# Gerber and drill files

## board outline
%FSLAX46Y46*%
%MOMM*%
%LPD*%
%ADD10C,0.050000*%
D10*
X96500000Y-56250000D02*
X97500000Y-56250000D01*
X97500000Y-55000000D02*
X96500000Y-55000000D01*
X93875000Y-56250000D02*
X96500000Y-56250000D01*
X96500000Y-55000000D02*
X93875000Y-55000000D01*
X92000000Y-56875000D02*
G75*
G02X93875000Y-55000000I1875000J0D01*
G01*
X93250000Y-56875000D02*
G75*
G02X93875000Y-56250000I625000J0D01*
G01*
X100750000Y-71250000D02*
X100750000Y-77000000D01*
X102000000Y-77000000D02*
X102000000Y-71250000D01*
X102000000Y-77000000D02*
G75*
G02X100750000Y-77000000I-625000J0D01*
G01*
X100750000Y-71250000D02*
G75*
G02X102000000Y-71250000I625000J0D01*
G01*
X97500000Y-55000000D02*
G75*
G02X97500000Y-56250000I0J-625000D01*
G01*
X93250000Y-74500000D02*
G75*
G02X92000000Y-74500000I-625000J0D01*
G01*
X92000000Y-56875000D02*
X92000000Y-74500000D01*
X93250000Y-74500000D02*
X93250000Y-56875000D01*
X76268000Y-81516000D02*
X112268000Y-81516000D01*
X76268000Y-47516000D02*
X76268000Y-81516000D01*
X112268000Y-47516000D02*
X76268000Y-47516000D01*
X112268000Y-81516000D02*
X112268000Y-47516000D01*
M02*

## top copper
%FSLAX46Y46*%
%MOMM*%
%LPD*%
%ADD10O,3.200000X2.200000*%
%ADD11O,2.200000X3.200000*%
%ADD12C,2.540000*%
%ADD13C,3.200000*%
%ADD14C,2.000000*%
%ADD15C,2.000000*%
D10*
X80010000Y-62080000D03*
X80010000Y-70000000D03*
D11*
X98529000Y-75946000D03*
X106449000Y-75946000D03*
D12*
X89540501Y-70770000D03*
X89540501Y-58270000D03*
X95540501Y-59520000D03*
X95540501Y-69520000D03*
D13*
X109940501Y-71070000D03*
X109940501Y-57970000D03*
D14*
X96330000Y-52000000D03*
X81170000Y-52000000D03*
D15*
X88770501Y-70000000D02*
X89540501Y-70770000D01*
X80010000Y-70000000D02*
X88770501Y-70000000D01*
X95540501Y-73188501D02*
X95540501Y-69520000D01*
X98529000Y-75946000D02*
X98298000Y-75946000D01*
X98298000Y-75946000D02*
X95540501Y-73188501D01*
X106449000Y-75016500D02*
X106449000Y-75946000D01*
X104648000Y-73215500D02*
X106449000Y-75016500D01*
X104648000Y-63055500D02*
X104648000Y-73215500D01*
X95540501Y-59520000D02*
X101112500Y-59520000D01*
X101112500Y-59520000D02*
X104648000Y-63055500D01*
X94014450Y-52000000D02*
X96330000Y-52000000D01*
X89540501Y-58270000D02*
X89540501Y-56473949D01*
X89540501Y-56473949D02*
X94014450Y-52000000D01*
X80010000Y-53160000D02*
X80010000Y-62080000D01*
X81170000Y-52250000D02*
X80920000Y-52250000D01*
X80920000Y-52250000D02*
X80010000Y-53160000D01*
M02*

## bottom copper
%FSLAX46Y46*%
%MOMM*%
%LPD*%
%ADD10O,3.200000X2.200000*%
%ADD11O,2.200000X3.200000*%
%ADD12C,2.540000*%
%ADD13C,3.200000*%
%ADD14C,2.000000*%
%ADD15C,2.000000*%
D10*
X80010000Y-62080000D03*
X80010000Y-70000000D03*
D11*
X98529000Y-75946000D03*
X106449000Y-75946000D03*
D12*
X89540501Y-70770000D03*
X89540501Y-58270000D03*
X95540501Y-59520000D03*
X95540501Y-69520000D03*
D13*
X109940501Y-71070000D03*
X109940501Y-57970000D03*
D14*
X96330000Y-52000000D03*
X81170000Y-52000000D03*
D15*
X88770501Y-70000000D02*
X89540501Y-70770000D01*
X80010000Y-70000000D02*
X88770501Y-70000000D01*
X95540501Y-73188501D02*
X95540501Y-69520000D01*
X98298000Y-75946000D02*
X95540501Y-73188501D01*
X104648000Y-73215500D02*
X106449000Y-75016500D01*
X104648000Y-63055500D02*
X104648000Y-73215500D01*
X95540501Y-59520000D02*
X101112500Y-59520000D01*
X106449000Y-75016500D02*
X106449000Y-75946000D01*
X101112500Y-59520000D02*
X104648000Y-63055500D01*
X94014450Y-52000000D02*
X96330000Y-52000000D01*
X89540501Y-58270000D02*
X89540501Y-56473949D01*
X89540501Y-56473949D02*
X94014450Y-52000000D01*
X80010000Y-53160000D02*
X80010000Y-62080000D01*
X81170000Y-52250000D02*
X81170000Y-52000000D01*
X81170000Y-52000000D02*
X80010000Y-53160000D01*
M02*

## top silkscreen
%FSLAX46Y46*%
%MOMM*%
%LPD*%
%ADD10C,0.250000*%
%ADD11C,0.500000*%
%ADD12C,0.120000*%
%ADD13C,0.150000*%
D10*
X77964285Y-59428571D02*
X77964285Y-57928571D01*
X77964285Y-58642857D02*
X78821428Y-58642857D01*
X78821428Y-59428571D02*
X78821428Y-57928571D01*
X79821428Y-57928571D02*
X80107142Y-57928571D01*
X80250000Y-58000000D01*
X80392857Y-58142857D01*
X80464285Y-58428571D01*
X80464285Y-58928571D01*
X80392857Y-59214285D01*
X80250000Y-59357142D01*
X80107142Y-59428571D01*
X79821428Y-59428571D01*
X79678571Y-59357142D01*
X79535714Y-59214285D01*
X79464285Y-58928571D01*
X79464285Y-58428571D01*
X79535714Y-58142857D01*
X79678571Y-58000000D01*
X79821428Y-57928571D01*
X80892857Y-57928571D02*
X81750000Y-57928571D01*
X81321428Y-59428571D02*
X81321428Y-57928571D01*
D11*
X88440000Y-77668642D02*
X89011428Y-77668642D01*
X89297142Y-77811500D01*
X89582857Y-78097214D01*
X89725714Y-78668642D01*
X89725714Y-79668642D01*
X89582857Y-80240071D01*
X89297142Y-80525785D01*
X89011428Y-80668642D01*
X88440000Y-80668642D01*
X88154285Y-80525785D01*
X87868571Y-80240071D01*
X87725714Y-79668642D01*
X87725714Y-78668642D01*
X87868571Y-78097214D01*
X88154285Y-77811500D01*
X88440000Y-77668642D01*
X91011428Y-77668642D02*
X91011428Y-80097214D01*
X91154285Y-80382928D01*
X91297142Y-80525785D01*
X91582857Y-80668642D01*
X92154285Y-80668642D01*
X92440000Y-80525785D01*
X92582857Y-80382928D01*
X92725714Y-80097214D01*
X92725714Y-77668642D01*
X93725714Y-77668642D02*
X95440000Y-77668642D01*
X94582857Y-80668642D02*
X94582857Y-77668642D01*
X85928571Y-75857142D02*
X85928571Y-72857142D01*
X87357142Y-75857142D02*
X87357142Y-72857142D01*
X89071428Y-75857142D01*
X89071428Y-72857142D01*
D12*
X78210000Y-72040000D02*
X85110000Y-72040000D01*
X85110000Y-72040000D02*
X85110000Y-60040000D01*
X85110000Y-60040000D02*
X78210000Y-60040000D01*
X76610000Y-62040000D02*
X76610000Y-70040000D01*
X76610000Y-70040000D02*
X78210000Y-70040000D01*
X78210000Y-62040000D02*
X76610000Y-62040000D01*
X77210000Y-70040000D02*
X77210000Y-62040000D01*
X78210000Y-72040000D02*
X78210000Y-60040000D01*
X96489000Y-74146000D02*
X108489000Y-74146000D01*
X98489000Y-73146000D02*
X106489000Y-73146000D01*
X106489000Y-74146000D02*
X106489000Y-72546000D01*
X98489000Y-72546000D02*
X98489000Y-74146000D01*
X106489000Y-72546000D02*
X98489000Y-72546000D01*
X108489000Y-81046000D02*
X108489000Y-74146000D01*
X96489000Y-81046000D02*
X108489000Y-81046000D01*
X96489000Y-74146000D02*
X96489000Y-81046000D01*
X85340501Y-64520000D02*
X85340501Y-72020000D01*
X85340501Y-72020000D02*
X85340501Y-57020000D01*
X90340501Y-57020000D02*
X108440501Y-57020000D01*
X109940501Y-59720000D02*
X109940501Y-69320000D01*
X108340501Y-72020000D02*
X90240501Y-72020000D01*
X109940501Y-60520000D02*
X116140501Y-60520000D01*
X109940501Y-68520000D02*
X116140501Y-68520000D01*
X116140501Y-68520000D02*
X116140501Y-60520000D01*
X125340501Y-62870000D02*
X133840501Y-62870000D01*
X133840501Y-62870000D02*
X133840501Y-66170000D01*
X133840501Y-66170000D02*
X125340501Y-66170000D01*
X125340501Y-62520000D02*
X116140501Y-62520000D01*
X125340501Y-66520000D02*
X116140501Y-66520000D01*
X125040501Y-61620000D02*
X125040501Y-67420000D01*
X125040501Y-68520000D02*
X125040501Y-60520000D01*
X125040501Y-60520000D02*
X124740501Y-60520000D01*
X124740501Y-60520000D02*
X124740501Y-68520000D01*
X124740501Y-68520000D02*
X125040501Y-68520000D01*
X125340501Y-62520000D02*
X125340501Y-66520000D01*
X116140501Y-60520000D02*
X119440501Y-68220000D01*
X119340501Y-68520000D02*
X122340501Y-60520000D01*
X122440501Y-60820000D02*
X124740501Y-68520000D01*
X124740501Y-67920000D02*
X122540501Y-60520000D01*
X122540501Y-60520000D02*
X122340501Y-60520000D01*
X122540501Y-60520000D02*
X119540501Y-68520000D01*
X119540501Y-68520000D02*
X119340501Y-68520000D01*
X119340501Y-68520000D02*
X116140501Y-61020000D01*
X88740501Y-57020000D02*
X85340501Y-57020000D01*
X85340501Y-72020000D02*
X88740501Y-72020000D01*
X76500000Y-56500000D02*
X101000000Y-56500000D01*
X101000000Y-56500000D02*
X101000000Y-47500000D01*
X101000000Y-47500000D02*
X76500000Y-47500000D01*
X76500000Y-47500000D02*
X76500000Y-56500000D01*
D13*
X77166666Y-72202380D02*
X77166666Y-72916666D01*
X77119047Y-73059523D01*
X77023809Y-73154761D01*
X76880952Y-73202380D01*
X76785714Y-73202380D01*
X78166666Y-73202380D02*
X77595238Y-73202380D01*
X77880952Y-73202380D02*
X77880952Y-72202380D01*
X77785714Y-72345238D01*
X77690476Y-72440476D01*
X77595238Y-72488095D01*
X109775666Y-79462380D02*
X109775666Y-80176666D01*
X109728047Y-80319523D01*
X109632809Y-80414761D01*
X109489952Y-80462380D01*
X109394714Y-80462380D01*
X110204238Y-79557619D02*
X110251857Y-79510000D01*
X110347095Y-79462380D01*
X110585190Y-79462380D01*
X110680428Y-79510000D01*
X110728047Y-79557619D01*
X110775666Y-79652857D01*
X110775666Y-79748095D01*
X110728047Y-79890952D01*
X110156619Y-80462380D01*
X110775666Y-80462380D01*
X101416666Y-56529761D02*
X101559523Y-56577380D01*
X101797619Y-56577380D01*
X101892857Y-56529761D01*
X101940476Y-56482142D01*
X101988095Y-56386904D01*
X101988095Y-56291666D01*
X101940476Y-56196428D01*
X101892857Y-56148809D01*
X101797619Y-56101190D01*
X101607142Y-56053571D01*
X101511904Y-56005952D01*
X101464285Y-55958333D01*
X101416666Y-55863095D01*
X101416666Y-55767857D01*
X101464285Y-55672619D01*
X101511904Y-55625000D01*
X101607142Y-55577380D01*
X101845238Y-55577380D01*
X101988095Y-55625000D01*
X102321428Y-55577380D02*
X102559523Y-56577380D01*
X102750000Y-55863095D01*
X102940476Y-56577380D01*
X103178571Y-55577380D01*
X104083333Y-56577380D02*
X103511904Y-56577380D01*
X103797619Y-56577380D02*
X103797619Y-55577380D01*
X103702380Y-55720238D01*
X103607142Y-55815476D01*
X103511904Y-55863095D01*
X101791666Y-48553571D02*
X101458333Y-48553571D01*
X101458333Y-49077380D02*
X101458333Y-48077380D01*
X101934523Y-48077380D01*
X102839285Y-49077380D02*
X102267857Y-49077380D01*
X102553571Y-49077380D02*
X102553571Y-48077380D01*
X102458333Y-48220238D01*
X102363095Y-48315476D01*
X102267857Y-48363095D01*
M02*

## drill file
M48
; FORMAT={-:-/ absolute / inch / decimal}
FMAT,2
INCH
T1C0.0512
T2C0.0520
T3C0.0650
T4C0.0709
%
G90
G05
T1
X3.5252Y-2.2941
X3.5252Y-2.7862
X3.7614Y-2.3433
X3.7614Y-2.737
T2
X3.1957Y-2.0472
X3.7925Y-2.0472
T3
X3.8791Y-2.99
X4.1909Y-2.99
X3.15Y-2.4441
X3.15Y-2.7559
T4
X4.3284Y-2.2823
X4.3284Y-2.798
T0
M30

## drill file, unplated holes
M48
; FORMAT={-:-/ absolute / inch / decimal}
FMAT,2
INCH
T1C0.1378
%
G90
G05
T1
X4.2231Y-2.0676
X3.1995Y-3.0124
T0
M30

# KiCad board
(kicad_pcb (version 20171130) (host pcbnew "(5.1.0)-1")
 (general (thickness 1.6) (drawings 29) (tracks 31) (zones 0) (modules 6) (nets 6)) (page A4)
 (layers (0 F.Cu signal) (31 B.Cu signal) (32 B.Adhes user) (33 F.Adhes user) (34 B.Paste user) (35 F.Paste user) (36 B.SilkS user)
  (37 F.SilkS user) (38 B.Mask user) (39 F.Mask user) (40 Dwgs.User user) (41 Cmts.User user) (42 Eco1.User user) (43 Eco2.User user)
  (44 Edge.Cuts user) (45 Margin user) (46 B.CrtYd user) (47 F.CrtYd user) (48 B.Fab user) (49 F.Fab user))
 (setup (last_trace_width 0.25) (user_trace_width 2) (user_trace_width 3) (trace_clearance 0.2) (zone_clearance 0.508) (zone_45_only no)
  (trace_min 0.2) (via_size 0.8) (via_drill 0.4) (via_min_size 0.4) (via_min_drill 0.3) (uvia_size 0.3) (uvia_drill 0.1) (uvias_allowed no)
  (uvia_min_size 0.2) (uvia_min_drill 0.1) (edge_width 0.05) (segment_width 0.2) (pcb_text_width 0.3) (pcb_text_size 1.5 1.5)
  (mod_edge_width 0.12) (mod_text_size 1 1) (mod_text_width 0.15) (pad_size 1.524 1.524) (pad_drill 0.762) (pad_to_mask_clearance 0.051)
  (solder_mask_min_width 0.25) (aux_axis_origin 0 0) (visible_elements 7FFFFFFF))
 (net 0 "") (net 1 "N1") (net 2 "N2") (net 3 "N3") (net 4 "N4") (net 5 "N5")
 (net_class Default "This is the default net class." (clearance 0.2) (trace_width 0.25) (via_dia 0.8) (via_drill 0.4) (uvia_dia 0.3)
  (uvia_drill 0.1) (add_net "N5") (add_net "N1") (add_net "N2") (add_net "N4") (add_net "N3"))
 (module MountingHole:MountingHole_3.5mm (layer F.Cu) (at 107.268 52.516)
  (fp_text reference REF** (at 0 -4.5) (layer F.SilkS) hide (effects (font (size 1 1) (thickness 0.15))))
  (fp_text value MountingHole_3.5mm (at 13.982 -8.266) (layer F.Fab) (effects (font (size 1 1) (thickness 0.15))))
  (pad 1 np_thru_hole circle (at 0 0) (size 3.5 3.5) (drill 3.5) (layers *.Cu *.Mask)))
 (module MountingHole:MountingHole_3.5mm (layer F.Cu) (at 81.268 76.516)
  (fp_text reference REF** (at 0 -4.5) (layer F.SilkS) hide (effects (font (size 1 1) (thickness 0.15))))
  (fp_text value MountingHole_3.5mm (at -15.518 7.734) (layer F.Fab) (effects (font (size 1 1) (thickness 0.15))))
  (pad 1 np_thru_hole circle (at 0 0) (size 3.5 3.5) (drill 3.5) (layers *.Cu *.Mask)))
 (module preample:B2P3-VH (layer F.Cu) (at 80.01 66.04 270)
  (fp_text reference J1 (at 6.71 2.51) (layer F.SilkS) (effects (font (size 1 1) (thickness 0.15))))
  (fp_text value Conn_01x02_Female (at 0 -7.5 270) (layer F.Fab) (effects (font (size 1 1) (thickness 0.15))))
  (fp_line (start 6 1.8) (end 6 -5.1) (layer F.SilkS) (width 0.12))
  (fp_line (start 6 -5.1) (end -6 -5.1) (layer F.SilkS) (width 0.12))
  (fp_line (start -6 -5.1) (end -6 1.8) (layer F.SilkS) (width 0.12))
  (fp_line (start -4 3.4) (end 4 3.4) (layer F.SilkS) (width 0.12))
  (fp_line (start 4 3.4) (end 4 1.8) (layer F.SilkS) (width 0.12))
  (fp_line (start -4 1.8) (end -4 3.4) (layer F.SilkS) (width 0.12))
  (fp_line (start 4 2.8) (end -4 2.8) (layer F.SilkS) (width 0.12))
  (fp_line (start 6 1.8) (end -6 1.8) (layer F.SilkS) (width 0.12))
  (pad 1 thru_hole oval (at -3.96 0 270) (size 2.2 3.2) (drill 1.65) (layers *.Cu *.Mask) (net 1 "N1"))
  (pad 2 thru_hole oval (at 3.96 0 270) (size 2.2 3.2) (drill 1.65) (layers *.Cu *.Mask) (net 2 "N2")))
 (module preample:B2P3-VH (layer F.Cu) (at 102.489 75.946 180)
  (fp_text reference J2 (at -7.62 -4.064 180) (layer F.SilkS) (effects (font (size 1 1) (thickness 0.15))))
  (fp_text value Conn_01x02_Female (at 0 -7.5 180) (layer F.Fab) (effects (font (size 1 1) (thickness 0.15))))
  (fp_line (start 6 1.8) (end -6 1.8) (layer F.SilkS) (width 0.12))
  (fp_line (start 4 2.8) (end -4 2.8) (layer F.SilkS) (width 0.12))
  (fp_line (start -4 1.8) (end -4 3.4) (layer F.SilkS) (width 0.12))
  (fp_line (start 4 3.4) (end 4 1.8) (layer F.SilkS) (width 0.12))
  (fp_line (start -4 3.4) (end 4 3.4) (layer F.SilkS) (width 0.12))
  (fp_line (start -6 -5.1) (end -6 1.8) (layer F.SilkS) (width 0.12))
  (fp_line (start 6 -5.1) (end -6 -5.1) (layer F.SilkS) (width 0.12))
  (fp_line (start 6 1.8) (end 6 -5.1) (layer F.SilkS) (width 0.12))
  (pad 2 thru_hole oval (at 3.96 0 180) (size 2.2 3.2) (drill 1.65) (layers *.Cu *.Mask) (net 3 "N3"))
  (pad 1 thru_hole oval (at -3.96 0 180) (size 2.2 3.2) (drill 1.65) (layers *.Cu *.Mask) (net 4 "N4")))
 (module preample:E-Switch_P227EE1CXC (layer F.Cu) (at 99.740501 64.52)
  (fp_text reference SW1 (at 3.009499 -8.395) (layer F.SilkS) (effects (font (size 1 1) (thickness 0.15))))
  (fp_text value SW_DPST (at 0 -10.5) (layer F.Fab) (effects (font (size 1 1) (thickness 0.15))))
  (fp_line (start -14.4 0) (end -14.4 7.5) (layer F.SilkS) (width 0.12))
  (fp_line (start -14.4 7.5) (end -14.4 -7.5) (layer F.SilkS) (width 0.12))
  (fp_line (start -9.4 -7.5) (end 8.7 -7.5) (layer F.SilkS) (width 0.12))
  (fp_line (start 10.2 -4.8) (end 10.2 4.8) (layer F.SilkS) (width 0.12))
  (fp_line (start 8.6 7.5) (end -9.5 7.5) (layer F.SilkS) (width 0.12))
  (fp_line (start 10.2 -4) (end 16.4 -4) (layer F.SilkS) (width 0.12))
  (fp_line (start 10.2 4) (end 16.4 4) (layer F.SilkS) (width 0.12))
  (fp_line (start 16.4 4) (end 16.4 -4) (layer F.SilkS) (width 0.12))
  (fp_line (start 25.6 -1.65) (end 34.1 -1.65) (layer F.SilkS) (width 0.12))
  (fp_line (start 34.1 -1.65) (end 34.1 1.65) (layer F.SilkS) (width 0.12))
  (fp_line (start 34.1 1.65) (end 25.6 1.65) (layer F.SilkS) (width 0.12))
  (fp_line (start 25.6 -2) (end 16.4 -2) (layer F.SilkS) (width 0.12))
  (fp_line (start 25.6 2) (end 16.4 2) (layer F.SilkS) (width 0.12))
  (fp_line (start 25.3 -2.9) (end 25.3 2.9) (layer F.SilkS) (width 0.12))
  (fp_line (start 25.3 4) (end 25.3 -4) (layer F.SilkS) (width 0.12))
  (fp_line (start 25.3 -4) (end 25 -4) (layer F.SilkS) (width 0.12))
  (fp_line (start 25 -4) (end 25 4) (layer F.SilkS) (width 0.12))
  (fp_line (start 25 4) (end 25.3 4) (layer F.SilkS) (width 0.12))
  (fp_line (start 25.6 -2) (end 25.6 2) (layer F.SilkS) (width 0.12))
  (fp_line (start 16.4 -4) (end 19.7 3.7) (layer F.SilkS) (width 0.12))
  (fp_line (start 19.6 4) (end 22.6 -4) (layer F.SilkS) (width 0.12))
  (fp_line (start 22.7 -3.7) (end 25 4) (layer F.SilkS) (width 0.12))
  (fp_line (start 25 3.4) (end 22.8 -4) (layer F.SilkS) (width 0.12))
  (fp_line (start 22.8 -4) (end 22.6 -4) (layer F.SilkS) (width 0.12))
  (fp_line (start 22.8 -4) (end 19.8 4) (layer F.SilkS) (width 0.12))
  (fp_line (start 19.8 4) (end 19.6 4) (layer F.SilkS) (width 0.12))
  (fp_line (start 19.6 4) (end 16.4 -3.5) (layer F.SilkS) (width 0.12))
  (fp_line (start -11 -7.5) (end -14.4 -7.5) (layer F.SilkS) (width 0.12))
  (fp_line (start -14.4 7.5) (end -11 7.5) (layer F.SilkS) (width 0.12))
  (pad 3 thru_hole circle (at -10.2 6.25) (size 2.54 2.54) (drill 1.3) (layers *.Cu *.Mask) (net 2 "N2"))
  (pad 1 thru_hole circle (at -10.2 -6.25) (size 2.54 2.54) (drill 1.3) (layers *.Cu *.Mask) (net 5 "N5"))
  (pad 2 thru_hole circle (at -4.2 -5) (size 2.54 2.54) (drill 1.3) (layers *.Cu *.Mask) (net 4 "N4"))
  (pad 4 thru_hole circle (at -4.2 5) (size 2.54 2.54) (drill 1.3) (layers *.Cu *.Mask) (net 3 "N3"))
  (pad 0 thru_hole circle (at 10.2 6.55) (size 3.2 3.2) (drill 1.8) (layers *.Cu *.Mask))
  (pad 0 thru_hole circle (at 10.2 -6.55) (size 3.2 3.2) (drill 1.8) (layers *.Cu *.Mask)))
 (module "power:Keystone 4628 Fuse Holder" (layer F.Cu) (at 88.75 52 180)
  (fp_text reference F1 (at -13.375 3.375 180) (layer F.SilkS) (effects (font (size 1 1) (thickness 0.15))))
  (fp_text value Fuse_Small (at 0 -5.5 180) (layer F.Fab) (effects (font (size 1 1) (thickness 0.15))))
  (fp_line (start 12.25 -4.5) (end -12.25 -4.5) (layer F.SilkS) (width 0.12))
  (fp_line (start -12.25 -4.5) (end -12.25 4.5) (layer F.SilkS) (width 0.12))
  (fp_line (start -12.25 4.5) (end 12.25 4.5) (layer F.SilkS) (width 0.12))
  (fp_line (start 12.25 4.5) (end 12.25 -4.5) (layer F.SilkS) (width 0.12))
  (pad 1 thru_hole circle (at -7.58 0 180) (size 2 2) (drill 1.32) (layers *.Cu *.Mask) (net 5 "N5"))
  (pad 2 thru_hole circle (at 7.58 0 180) (size 2 2) (drill 1.32) (layers *.Cu *.Mask) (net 1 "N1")))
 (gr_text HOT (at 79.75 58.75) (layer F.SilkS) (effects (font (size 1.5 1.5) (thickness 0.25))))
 (gr_line (start 96.5 56.25) (end 97.5 56.25) (layer Edge.Cuts) (width 0.05))
 (gr_line (start 97.5 55) (end 96.5 55) (layer Edge.Cuts) (width 0.05))
 (gr_line (start 93.875 56.25) (end 96.5 56.25) (layer Edge.Cuts) (width 0.05))
 (gr_line (start 96.5 55) (end 93.875 55) (layer Edge.Cuts) (width 0.05))
 (gr_arc (start 93.875 56.875) (end 93.875 55) (angle -90) (layer Edge.Cuts) (width 0.05))
 (gr_arc (start 93.875 56.875) (end 93.875 56.25) (angle -90) (layer Edge.Cuts) (width 0.05))
 (gr_line (start 100.75 71.25) (end 100.75 77) (layer Edge.Cuts) (width 0.05))
 (gr_line (start 102 77) (end 102 71.25) (layer Edge.Cuts) (width 0.05))
 (gr_arc (start 101.375 77) (end 100.75 77) (angle -180) (layer Edge.Cuts) (width 0.05))
 (gr_arc (start 101.375 71.25) (end 102 71.25) (angle -180) (layer Edge.Cuts) (width 0.05))
 (gr_arc (start 97.5 55.625) (end 97.5 56.25) (angle -180) (layer Edge.Cuts) (width 0.05))
 (gr_arc (start 92.625 74.5) (end 92 74.5) (angle -180) (layer Edge.Cuts) (width 0.05))
 (gr_line (start 92 56.875) (end 92 74.5) (layer Edge.Cuts) (width 0.05))
 (gr_line (start 93.25 74.5) (end 93.25 56.875) (layer Edge.Cuts) (width 0.05))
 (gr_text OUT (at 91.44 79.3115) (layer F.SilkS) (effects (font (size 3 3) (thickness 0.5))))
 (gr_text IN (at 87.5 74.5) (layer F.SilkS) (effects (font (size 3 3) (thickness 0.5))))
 (gr_line (start 76.268 81.516) (end 112.268 81.516) (layer Edge.Cuts) (width 0.05))
 (gr_line (start 76.268 47.516) (end 76.268 81.516) (layer Edge.Cuts) (width 0.05))
 (gr_line (start 112.268 47.516) (end 76.268 47.516) (layer Edge.Cuts) (width 0.05))
 (gr_line (start 112.268 81.516) (end 112.268 47.516) (layer Edge.Cuts) (width 0.05))
 (segment (start 88.770501 70) (end 89.540501 70.77) (width 2) (layer B.Cu) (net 2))
 (segment (start 80.01 70) (end 88.770501 70) (width 2) (layer B.Cu) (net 2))
 (segment (start 88.770501 70) (end 89.540501 70.77) (width 2) (layer F.Cu) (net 2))
 (segment (start 80.01 70) (end 88.770501 70) (width 2) (layer F.Cu) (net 2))
 (segment (start 95.540501 73.188501) (end 95.540501 69.52) (width 2) (layer B.Cu) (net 3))
 (segment (start 98.298 75.946) (end 95.540501 73.188501) (width 2) (layer B.Cu) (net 3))
 (segment (start 95.540501 73.188501) (end 95.540501 69.52) (width 2) (layer F.Cu) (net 3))
 (segment (start 98.529 75.946) (end 98.298 75.946) (width 2) (layer F.Cu) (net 3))
 (segment (start 98.298 75.946) (end 95.540501 73.188501) (width 2) (layer F.Cu) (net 3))
 (segment (start 104.648 73.2155) (end 106.449 75.0165) (width 2) (layer B.Cu) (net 4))
 (segment (start 104.648 63.0555) (end 104.648 73.2155) (width 2) (layer B.Cu) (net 4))
 (segment (start 95.540501 59.52) (end 101.1125 59.52) (width 2) (layer B.Cu) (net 4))
 (segment (start 106.449 75.0165) (end 106.449 75.946) (width 2) (layer B.Cu) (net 4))
 (segment (start 101.1125 59.52) (end 104.648 63.0555) (width 2) (layer B.Cu) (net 4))
 (segment (start 106.449 75.0165) (end 106.449 75.946) (width 2) (layer F.Cu) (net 4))
 (segment (start 104.648 73.2155) (end 106.449 75.0165) (width 2) (layer F.Cu) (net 4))
 (segment (start 104.648 63.0555) (end 104.648 73.2155) (width 2) (layer F.Cu) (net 4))
 (segment (start 95.540501 59.52) (end 101.1125 59.52) (width 2) (layer F.Cu) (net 4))
 (segment (start 101.1125 59.52) (end 104.648 63.0555) (width 2) (layer F.Cu) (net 4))
 (segment (start 94.01445 52) (end 96.33 52) (width 2) (layer F.Cu) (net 5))
 (segment (start 89.540501 58.27) (end 89.540501 56.473949) (width 2) (layer F.Cu) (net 5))
 (segment (start 89.540501 56.473949) (end 94.01445 52) (width 2) (layer F.Cu) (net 5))
 (segment (start 94.01445 52) (end 96.33 52) (width 2) (layer B.Cu) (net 5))
 (segment (start 89.540501 58.27) (end 89.540501 56.473949) (width 2) (layer B.Cu) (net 5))
 (segment (start 89.540501 56.473949) (end 94.01445 52) (width 2) (layer B.Cu) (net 5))
 (segment (start 80.01 53.16) (end 80.01 62.08) (width 2) (layer F.Cu) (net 1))
 (segment (start 81.17 52.25) (end 80.92 52.25) (width 2) (layer F.Cu) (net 1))
 (segment (start 80.92 52.25) (end 80.01 53.16) (width 2) (layer F.Cu) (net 1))
 (segment (start 80.01 53.16) (end 80.01 62.08) (width 2) (layer B.Cu) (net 1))
 (segment (start 81.17 52.25) (end 81.17 52) (width 2) (layer B.Cu) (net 1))
 (segment (start 81.17 52) (end 80.01 53.16) (width 2) (layer B.Cu) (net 1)))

